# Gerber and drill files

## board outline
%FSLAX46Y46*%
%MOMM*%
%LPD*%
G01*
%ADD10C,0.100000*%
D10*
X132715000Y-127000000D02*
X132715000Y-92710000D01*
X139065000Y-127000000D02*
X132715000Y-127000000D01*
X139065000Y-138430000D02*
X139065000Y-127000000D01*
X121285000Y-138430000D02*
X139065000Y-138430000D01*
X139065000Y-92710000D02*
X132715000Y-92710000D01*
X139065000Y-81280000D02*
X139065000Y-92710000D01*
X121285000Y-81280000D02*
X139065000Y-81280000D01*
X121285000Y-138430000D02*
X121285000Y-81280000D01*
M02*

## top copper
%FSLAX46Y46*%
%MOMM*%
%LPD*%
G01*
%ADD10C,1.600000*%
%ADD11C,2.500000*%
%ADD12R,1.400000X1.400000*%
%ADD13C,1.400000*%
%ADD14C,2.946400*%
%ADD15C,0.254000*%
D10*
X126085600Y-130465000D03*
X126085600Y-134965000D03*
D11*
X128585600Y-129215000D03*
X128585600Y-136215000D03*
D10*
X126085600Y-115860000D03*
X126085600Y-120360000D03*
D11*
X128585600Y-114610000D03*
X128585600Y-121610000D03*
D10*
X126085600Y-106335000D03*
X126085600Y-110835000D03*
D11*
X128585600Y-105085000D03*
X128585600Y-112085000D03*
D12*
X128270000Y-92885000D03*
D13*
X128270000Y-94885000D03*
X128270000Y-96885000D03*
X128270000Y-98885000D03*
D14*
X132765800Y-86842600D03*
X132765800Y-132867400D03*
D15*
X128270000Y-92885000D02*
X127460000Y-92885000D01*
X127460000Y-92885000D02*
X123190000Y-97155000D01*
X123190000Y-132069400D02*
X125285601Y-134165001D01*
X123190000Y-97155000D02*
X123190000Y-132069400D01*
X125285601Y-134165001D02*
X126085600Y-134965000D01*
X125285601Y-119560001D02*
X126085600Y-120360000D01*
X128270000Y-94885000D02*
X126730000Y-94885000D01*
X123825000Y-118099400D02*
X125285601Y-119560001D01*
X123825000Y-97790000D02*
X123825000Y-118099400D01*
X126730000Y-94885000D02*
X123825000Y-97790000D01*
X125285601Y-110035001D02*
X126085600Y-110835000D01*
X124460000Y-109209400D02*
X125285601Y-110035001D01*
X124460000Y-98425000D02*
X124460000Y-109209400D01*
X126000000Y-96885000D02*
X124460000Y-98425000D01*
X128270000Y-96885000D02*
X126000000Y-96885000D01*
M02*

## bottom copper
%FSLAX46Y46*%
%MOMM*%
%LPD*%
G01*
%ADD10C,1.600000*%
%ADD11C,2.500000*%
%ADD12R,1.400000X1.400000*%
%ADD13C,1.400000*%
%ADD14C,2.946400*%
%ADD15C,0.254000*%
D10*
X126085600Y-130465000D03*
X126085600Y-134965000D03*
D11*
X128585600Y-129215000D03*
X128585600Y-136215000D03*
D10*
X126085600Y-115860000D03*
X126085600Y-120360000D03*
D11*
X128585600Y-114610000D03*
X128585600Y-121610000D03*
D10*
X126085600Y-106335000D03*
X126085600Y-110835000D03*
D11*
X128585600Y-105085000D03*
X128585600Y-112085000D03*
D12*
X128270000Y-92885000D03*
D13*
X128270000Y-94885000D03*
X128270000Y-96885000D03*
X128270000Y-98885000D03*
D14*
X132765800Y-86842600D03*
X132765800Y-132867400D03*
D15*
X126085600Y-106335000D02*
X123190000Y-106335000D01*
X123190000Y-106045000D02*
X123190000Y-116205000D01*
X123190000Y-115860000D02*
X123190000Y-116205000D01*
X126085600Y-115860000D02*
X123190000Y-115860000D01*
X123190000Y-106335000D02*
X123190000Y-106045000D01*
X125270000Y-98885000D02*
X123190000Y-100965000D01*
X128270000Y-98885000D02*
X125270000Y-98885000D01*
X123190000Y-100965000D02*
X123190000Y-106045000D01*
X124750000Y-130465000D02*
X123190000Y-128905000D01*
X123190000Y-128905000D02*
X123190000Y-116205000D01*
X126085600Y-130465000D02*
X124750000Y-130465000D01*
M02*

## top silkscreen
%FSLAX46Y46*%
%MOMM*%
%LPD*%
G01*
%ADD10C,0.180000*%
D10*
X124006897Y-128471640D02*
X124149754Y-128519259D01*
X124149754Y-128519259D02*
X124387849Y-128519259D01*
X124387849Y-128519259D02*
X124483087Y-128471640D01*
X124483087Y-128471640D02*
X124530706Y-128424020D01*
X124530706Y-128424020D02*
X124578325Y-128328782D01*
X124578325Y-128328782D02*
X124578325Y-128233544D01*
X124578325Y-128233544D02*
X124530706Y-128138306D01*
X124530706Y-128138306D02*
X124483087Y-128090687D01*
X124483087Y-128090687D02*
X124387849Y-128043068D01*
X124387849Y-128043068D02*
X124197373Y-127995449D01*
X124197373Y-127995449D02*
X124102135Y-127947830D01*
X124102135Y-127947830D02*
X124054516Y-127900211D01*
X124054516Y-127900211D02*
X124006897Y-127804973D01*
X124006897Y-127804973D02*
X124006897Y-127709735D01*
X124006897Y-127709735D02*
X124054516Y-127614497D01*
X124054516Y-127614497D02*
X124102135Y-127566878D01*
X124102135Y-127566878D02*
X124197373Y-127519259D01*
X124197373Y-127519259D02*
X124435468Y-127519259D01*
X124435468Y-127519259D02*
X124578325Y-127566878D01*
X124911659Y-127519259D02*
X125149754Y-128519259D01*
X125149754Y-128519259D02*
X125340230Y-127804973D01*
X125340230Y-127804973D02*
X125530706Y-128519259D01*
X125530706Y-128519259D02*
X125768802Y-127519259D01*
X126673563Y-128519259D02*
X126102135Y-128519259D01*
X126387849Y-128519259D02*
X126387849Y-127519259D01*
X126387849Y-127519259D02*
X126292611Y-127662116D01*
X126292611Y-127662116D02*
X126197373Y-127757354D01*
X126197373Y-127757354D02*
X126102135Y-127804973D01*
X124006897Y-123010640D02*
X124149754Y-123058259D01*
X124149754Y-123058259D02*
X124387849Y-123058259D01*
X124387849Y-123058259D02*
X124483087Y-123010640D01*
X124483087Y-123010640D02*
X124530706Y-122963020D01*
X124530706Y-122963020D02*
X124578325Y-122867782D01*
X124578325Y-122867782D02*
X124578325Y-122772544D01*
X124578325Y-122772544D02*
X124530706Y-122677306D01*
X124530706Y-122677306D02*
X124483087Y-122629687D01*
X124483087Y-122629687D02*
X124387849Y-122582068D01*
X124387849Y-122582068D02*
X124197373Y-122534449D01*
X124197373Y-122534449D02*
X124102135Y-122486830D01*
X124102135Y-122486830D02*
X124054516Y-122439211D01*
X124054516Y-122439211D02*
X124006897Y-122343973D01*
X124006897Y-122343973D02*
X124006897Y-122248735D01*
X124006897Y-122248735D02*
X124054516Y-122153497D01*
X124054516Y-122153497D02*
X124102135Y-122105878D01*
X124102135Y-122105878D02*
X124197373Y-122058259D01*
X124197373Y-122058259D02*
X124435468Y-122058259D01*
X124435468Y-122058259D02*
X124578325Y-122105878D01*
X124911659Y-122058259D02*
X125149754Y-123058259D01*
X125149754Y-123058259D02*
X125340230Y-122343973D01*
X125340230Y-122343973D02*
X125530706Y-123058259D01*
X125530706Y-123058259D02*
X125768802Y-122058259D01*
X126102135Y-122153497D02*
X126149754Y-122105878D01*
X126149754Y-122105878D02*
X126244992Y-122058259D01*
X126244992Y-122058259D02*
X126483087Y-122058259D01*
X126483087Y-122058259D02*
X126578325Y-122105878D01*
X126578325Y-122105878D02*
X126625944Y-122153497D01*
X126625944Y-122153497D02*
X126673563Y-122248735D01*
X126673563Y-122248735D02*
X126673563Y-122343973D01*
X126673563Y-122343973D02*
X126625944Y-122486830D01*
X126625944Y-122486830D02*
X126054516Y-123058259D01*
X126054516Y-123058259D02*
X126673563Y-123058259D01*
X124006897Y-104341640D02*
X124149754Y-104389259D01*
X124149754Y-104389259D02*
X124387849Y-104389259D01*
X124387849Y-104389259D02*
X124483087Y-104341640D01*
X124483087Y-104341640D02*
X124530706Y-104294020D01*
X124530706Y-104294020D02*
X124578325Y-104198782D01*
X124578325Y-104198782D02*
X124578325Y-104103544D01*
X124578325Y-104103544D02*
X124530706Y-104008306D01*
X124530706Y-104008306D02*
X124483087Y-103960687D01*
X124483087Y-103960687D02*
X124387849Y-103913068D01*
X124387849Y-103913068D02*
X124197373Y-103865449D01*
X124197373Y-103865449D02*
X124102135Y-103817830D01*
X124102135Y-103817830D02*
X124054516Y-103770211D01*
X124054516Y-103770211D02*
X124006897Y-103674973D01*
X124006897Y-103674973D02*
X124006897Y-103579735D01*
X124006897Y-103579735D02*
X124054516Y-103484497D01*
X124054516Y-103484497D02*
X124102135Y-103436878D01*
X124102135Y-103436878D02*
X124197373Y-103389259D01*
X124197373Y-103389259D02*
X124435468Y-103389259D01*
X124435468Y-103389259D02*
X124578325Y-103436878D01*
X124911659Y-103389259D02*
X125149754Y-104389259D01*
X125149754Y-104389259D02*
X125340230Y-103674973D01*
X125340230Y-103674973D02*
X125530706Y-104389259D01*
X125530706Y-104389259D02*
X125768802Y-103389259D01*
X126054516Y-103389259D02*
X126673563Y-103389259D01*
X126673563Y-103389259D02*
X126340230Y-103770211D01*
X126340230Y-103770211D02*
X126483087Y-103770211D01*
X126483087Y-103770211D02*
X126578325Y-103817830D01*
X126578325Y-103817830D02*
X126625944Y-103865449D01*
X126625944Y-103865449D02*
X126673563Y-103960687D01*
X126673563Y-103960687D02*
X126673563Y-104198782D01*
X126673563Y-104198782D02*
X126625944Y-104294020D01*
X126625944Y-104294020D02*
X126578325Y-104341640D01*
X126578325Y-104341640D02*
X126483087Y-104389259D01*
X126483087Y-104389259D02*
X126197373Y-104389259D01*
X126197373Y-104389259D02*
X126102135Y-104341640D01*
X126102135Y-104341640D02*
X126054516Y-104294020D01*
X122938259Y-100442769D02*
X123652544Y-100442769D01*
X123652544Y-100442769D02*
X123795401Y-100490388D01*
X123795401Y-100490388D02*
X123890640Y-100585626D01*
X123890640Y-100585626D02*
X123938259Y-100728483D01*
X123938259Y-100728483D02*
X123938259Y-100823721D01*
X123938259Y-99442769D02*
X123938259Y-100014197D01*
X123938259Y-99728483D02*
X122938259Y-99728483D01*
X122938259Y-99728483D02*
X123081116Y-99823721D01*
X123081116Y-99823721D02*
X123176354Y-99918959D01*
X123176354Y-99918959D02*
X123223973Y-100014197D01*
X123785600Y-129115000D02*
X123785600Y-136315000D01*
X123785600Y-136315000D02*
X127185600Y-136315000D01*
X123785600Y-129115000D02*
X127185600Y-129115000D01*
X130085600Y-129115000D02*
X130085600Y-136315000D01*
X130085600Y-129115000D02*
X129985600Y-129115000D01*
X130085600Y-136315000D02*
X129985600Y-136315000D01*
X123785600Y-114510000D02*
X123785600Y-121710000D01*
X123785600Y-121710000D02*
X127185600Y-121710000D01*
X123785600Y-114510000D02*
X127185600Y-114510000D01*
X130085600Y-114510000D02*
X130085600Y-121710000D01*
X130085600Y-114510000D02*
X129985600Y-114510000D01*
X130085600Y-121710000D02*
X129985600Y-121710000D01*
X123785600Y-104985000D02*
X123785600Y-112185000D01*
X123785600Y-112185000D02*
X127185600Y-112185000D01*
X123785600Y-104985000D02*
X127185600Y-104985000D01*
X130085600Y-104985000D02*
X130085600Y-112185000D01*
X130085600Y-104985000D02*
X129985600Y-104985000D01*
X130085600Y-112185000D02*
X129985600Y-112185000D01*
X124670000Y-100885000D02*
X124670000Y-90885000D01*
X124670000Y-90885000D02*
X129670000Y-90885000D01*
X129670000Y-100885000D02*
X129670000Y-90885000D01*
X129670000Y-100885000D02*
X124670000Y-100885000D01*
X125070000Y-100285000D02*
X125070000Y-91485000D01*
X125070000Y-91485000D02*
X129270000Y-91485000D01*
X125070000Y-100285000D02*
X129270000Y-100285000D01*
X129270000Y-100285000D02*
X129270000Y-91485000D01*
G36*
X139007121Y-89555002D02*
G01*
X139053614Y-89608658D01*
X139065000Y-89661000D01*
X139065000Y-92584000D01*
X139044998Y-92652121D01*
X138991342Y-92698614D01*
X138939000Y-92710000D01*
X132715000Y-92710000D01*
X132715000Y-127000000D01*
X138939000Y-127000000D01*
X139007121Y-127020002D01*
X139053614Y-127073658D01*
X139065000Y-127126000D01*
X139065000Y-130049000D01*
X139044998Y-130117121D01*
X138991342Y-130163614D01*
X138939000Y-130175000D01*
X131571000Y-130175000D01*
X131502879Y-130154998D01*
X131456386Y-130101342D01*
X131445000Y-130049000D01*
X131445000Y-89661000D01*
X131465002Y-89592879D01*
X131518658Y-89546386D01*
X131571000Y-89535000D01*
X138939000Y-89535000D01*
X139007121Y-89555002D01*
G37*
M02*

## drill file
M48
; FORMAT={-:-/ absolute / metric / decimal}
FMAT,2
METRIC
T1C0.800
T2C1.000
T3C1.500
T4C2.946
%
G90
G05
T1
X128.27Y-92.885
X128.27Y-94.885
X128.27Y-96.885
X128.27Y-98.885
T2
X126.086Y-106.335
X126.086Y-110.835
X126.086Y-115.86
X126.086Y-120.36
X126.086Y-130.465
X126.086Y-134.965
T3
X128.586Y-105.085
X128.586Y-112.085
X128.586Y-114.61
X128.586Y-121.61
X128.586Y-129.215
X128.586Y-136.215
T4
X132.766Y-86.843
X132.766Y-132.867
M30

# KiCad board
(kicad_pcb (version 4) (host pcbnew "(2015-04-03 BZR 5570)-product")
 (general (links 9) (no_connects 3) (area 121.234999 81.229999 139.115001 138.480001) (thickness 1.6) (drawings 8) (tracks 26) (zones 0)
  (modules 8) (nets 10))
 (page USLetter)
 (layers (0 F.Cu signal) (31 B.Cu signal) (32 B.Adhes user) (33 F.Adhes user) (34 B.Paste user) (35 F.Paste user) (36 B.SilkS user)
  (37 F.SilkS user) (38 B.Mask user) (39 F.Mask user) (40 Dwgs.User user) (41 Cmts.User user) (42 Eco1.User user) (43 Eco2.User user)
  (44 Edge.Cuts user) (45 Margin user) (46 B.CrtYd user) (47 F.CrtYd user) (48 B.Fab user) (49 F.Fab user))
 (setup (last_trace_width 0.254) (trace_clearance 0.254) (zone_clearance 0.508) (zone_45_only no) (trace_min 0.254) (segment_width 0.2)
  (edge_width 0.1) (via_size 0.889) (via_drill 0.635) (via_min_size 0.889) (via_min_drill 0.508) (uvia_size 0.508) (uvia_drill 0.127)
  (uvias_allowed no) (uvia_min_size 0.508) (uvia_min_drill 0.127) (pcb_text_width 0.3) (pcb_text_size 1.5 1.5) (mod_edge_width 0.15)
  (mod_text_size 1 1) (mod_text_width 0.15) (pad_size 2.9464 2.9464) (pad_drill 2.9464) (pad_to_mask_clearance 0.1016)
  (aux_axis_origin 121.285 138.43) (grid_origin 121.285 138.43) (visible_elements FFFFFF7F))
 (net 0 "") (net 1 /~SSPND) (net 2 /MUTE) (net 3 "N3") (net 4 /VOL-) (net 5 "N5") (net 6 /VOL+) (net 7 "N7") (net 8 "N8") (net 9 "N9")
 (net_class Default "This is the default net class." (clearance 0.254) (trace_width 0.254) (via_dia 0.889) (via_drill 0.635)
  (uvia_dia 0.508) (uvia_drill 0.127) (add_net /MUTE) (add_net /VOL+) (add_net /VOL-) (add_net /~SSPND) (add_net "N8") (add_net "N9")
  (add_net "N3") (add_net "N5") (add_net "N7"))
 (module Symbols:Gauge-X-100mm (layer B.Cu) (at 108.585 151.13 90)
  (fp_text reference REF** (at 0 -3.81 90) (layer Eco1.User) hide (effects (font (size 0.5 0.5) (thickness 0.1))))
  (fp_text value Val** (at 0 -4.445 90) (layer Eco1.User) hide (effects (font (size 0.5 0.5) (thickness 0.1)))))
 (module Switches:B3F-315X (layer F.Cu) (at 126.0856 132.715 270)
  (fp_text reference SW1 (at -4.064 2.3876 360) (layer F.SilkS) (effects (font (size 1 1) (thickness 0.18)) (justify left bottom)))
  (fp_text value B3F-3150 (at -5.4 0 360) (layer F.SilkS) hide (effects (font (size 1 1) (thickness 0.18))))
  (fp_line (start -3.6 2.3) (end 3.6 2.3) (layer F.SilkS) (width 0.18))
  (fp_line (start 3.6 2.3) (end 3.6 -1.1) (layer F.SilkS) (width 0.18))
  (fp_line (start -3.6 2.3) (end -3.6 -1.1) (layer F.SilkS) (width 0.18))
  (fp_line (start -3.6 -4) (end 3.6 -4) (layer F.SilkS) (width 0.18))
  (fp_line (start -3.6 -4) (end -3.6 -3.9) (layer F.SilkS) (width 0.18))
  (fp_line (start 3.6 -4) (end 3.6 -3.9) (layer F.SilkS) (width 0.18))
  (pad 1 thru_hole circle (at -2.25 0 270) (size 1.6 1.6) (drill 1) (layers *.Cu *.Mask) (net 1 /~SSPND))
  (pad 2 thru_hole circle (at 2.25 0 270) (size 1.6 1.6) (drill 1) (layers *.Cu *.Mask) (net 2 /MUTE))
  (pad GND thru_hole circle (at -3.5 -2.5 270) (size 2.5 2.5) (drill 1.5) (layers *.Cu *.Mask) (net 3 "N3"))
  (pad GND thru_hole circle (at 3.5 -2.5 270) (size 2.5 2.5) (drill 1.5) (layers *.Cu *.Mask) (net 3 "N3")))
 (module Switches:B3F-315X (layer F.Cu) (at 126.0856 118.11 270)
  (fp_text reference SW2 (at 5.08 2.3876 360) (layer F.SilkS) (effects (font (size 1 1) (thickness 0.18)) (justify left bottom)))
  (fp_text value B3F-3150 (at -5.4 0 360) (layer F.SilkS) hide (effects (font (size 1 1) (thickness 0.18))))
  (fp_line (start -3.6 2.3) (end 3.6 2.3) (layer F.SilkS) (width 0.18))
  (fp_line (start 3.6 2.3) (end 3.6 -1.1) (layer F.SilkS) (width 0.18))
  (fp_line (start -3.6 2.3) (end -3.6 -1.1) (layer F.SilkS) (width 0.18))
  (fp_line (start -3.6 -4) (end 3.6 -4) (layer F.SilkS) (width 0.18))
  (fp_line (start -3.6 -4) (end -3.6 -3.9) (layer F.SilkS) (width 0.18))
  (fp_line (start 3.6 -4) (end 3.6 -3.9) (layer F.SilkS) (width 0.18))
  (pad 1 thru_hole circle (at -2.25 0 270) (size 1.6 1.6) (drill 1) (layers *.Cu *.Mask) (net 1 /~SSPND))
  (pad 2 thru_hole circle (at 2.25 0 270) (size 1.6 1.6) (drill 1) (layers *.Cu *.Mask) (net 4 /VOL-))
  (pad GND thru_hole circle (at -3.5 -2.5 270) (size 2.5 2.5) (drill 1.5) (layers *.Cu *.Mask) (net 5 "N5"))
  (pad GND thru_hole circle (at 3.5 -2.5 270) (size 2.5 2.5) (drill 1.5) (layers *.Cu *.Mask) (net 5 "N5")))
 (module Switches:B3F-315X (layer F.Cu) (at 126.0856 108.585 270)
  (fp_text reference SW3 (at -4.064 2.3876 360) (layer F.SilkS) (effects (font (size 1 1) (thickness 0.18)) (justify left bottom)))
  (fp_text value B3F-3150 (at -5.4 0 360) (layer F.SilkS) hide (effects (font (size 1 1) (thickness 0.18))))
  (fp_line (start -3.6 2.3) (end 3.6 2.3) (layer F.SilkS) (width 0.18))
  (fp_line (start 3.6 2.3) (end 3.6 -1.1) (layer F.SilkS) (width 0.18))
  (fp_line (start -3.6 2.3) (end -3.6 -1.1) (layer F.SilkS) (width 0.18))
  (fp_line (start -3.6 -4) (end 3.6 -4) (layer F.SilkS) (width 0.18))
  (fp_line (start -3.6 -4) (end -3.6 -3.9) (layer F.SilkS) (width 0.18))
  (fp_line (start 3.6 -4) (end 3.6 -3.9) (layer F.SilkS) (width 0.18))
  (pad 1 thru_hole circle (at -2.25 0 270) (size 1.6 1.6) (drill 1) (layers *.Cu *.Mask) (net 1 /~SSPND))
  (pad 2 thru_hole circle (at 2.25 0 270) (size 1.6 1.6) (drill 1) (layers *.Cu *.Mask) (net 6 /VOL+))
  (pad GND thru_hole circle (at -3.5 -2.5 270) (size 2.5 2.5) (drill 1.5) (layers *.Cu *.Mask) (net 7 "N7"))
  (pad GND thru_hole circle (at 3.5 -2.5 270) (size 2.5 2.5) (drill 1.5) (layers *.Cu *.Mask) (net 7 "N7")))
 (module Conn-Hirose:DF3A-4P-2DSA (layer F.Cu) (at 128.27 95.885 90)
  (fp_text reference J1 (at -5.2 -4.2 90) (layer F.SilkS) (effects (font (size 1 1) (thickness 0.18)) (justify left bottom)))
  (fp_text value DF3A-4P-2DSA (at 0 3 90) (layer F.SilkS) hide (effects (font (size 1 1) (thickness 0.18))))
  (fp_line (start -5 -3.6) (end 5 -3.6) (layer F.SilkS) (width 0.18))
  (fp_line (start 5 -3.6) (end 5 1.4) (layer F.SilkS) (width 0.18))
  (fp_line (start -5 1.4) (end 5 1.4) (layer F.SilkS) (width 0.18))
  (fp_line (start -5 1.4) (end -5 -3.6) (layer F.SilkS) (width 0.18))
  (fp_line (start -4.4 -3.2) (end 4.4 -3.2) (layer F.SilkS) (width 0.18))
  (fp_line (start 4.4 -3.2) (end 4.4 1) (layer F.SilkS) (width 0.18))
  (fp_line (start -4.4 -3.2) (end -4.4 1) (layer F.SilkS) (width 0.18))
  (fp_line (start -4.4 1) (end 4.4 1) (layer F.SilkS) (width 0.18))
  (pad 1 thru_hole rect (at 3 0 90) (size 1.4 1.4) (drill 0.8) (layers *.Cu *.Mask) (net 2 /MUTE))
  (pad 2 thru_hole circle (at 1 0 90) (size 1.4 1.4) (drill 0.8) (layers *.Cu *.Mask) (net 4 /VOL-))
  (pad 3 thru_hole circle (at -1 0 90) (size 1.4 1.4) (drill 0.8) (layers *.Cu *.Mask) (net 6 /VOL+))
  (pad 4 thru_hole circle (at -3 0 90) (size 1.4 1.4) (drill 0.8) (layers *.Cu *.Mask) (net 1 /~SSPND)))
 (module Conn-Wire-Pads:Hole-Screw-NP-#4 (layer F.Cu) (at 132.7658 86.8426)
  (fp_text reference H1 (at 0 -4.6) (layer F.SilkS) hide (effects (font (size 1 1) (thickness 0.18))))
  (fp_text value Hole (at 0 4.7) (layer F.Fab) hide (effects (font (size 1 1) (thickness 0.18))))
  (pad P thru_hole circle (at 0 0) (size 2.9464 2.9464) (drill 2.9464) (layers *.Cu *.Mask) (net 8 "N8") (clearance 2.7178) (zone_connect 0)))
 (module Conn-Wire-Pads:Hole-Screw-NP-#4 (layer F.Cu) (at 132.7658 132.8674)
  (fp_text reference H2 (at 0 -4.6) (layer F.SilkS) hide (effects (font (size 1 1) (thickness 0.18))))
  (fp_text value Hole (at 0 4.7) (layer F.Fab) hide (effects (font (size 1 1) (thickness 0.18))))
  (pad P thru_hole circle (at 0 0) (size 2.9464 2.9464) (drill 2.9464) (layers *.Cu *.Mask) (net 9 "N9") (clearance 2.7178) (zone_connect 0)))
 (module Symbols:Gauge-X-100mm (layer F.Cu) (at 108.585 151.13)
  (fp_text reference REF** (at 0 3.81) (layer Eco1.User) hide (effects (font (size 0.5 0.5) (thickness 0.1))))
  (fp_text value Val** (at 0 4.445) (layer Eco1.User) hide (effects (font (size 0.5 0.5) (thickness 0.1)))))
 (gr_line (start 132.715 127) (end 132.715 92.71) (angle 90) (layer Edge.Cuts) (width 0.1))
 (gr_line (start 139.065 127) (end 132.715 127) (angle 90) (layer Edge.Cuts) (width 0.1))
 (gr_line (start 139.065 138.43) (end 139.065 127) (angle 90) (layer Edge.Cuts) (width 0.1))
 (gr_line (start 121.285 138.43) (end 139.065 138.43) (angle 90) (layer Edge.Cuts) (width 0.1))
 (gr_line (start 139.065 92.71) (end 132.715 92.71) (angle 90) (layer Edge.Cuts) (width 0.1))
 (gr_line (start 139.065 81.28) (end 139.065 92.71) (angle 90) (layer Edge.Cuts) (width 0.1))
 (gr_line (start 121.285 81.28) (end 139.065 81.28) (angle 90) (layer Edge.Cuts) (width 0.1))
 (gr_line (start 121.285 138.43) (end 121.285 81.28) (angle 90) (layer Edge.Cuts) (width 0.1))
 (segment (start 126.0856 106.335) (end 123.19 106.335) (width 0.254) (layer B.Cu) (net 1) (status 10))
 (segment (start 123.19 106.045) (end 123.19 116.205) (width 0.254) (layer B.Cu) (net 1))
 (segment (start 123.19 115.86) (end 123.19 116.205) (width 0.254) (layer B.Cu) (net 1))
 (segment (start 126.0856 115.86) (end 123.19 115.86) (width 0.254) (layer B.Cu) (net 1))
 (segment (start 123.19 106.335) (end 123.19 106.045) (width 0.254) (layer B.Cu) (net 1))
 (segment (start 125.27 98.885) (end 123.19 100.965) (width 0.254) (layer B.Cu) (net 1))
 (segment (start 128.27 98.885) (end 125.27 98.885) (width 0.254) (layer B.Cu) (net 1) (status 10))
 (segment (start 123.19 100.965) (end 123.19 106.045) (width 0.254) (layer B.Cu) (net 1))
 (segment (start 124.75 130.465) (end 123.19 128.905) (width 0.254) (layer B.Cu) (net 1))
 (segment (start 123.19 128.905) (end 123.19 116.205) (width 0.254) (layer B.Cu) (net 1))
 (segment (start 126.0856 130.465) (end 124.75 130.465) (width 0.254) (layer B.Cu) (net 1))
 (segment (start 128.27 92.885) (end 127.46 92.885) (width 0.254) (layer F.Cu) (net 2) (status 10))
 (segment (start 127.46 92.885) (end 123.19 97.155) (width 0.254) (layer F.Cu) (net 2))
 (segment (start 123.19 132.0694) (end 125.285601 134.165001) (width 0.254) (layer F.Cu) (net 2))
 (segment (start 123.19 97.155) (end 123.19 132.0694) (width 0.254) (layer F.Cu) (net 2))
 (segment (start 125.285601 134.165001) (end 126.0856 134.965) (width 0.254) (layer F.Cu) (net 2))
 (segment (start 125.285601 119.560001) (end 126.0856 120.36) (width 0.254) (layer F.Cu) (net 4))
 (segment (start 128.27 94.885) (end 126.73 94.885) (width 0.254) (layer F.Cu) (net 4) (status 10))
 (segment (start 123.825 118.0994) (end 125.285601 119.560001) (width 0.254) (layer F.Cu) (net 4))
 (segment (start 123.825 97.79) (end 123.825 118.0994) (width 0.254) (layer F.Cu) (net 4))
 (segment (start 126.73 94.885) (end 123.825 97.79) (width 0.254) (layer F.Cu) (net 4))
 (segment (start 125.285601 110.035001) (end 126.0856 110.835) (width 0.254) (layer F.Cu) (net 6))
 (segment (start 124.46 109.2094) (end 125.285601 110.035001) (width 0.254) (layer F.Cu) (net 6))
 (segment (start 124.46 98.425) (end 124.46 109.2094) (width 0.254) (layer F.Cu) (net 6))
 (segment (start 126 96.885) (end 124.46 98.425) (width 0.254) (layer F.Cu) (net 6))
 (segment (start 128.27 96.885) (end 126 96.885) (width 0.254) (layer F.Cu) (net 6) (status 10))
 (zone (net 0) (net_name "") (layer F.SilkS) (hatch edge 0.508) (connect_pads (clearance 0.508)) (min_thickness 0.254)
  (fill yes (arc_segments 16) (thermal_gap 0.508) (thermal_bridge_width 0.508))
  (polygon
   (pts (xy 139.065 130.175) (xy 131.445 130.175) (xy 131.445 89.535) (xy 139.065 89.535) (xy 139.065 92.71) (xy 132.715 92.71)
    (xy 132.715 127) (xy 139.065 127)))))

